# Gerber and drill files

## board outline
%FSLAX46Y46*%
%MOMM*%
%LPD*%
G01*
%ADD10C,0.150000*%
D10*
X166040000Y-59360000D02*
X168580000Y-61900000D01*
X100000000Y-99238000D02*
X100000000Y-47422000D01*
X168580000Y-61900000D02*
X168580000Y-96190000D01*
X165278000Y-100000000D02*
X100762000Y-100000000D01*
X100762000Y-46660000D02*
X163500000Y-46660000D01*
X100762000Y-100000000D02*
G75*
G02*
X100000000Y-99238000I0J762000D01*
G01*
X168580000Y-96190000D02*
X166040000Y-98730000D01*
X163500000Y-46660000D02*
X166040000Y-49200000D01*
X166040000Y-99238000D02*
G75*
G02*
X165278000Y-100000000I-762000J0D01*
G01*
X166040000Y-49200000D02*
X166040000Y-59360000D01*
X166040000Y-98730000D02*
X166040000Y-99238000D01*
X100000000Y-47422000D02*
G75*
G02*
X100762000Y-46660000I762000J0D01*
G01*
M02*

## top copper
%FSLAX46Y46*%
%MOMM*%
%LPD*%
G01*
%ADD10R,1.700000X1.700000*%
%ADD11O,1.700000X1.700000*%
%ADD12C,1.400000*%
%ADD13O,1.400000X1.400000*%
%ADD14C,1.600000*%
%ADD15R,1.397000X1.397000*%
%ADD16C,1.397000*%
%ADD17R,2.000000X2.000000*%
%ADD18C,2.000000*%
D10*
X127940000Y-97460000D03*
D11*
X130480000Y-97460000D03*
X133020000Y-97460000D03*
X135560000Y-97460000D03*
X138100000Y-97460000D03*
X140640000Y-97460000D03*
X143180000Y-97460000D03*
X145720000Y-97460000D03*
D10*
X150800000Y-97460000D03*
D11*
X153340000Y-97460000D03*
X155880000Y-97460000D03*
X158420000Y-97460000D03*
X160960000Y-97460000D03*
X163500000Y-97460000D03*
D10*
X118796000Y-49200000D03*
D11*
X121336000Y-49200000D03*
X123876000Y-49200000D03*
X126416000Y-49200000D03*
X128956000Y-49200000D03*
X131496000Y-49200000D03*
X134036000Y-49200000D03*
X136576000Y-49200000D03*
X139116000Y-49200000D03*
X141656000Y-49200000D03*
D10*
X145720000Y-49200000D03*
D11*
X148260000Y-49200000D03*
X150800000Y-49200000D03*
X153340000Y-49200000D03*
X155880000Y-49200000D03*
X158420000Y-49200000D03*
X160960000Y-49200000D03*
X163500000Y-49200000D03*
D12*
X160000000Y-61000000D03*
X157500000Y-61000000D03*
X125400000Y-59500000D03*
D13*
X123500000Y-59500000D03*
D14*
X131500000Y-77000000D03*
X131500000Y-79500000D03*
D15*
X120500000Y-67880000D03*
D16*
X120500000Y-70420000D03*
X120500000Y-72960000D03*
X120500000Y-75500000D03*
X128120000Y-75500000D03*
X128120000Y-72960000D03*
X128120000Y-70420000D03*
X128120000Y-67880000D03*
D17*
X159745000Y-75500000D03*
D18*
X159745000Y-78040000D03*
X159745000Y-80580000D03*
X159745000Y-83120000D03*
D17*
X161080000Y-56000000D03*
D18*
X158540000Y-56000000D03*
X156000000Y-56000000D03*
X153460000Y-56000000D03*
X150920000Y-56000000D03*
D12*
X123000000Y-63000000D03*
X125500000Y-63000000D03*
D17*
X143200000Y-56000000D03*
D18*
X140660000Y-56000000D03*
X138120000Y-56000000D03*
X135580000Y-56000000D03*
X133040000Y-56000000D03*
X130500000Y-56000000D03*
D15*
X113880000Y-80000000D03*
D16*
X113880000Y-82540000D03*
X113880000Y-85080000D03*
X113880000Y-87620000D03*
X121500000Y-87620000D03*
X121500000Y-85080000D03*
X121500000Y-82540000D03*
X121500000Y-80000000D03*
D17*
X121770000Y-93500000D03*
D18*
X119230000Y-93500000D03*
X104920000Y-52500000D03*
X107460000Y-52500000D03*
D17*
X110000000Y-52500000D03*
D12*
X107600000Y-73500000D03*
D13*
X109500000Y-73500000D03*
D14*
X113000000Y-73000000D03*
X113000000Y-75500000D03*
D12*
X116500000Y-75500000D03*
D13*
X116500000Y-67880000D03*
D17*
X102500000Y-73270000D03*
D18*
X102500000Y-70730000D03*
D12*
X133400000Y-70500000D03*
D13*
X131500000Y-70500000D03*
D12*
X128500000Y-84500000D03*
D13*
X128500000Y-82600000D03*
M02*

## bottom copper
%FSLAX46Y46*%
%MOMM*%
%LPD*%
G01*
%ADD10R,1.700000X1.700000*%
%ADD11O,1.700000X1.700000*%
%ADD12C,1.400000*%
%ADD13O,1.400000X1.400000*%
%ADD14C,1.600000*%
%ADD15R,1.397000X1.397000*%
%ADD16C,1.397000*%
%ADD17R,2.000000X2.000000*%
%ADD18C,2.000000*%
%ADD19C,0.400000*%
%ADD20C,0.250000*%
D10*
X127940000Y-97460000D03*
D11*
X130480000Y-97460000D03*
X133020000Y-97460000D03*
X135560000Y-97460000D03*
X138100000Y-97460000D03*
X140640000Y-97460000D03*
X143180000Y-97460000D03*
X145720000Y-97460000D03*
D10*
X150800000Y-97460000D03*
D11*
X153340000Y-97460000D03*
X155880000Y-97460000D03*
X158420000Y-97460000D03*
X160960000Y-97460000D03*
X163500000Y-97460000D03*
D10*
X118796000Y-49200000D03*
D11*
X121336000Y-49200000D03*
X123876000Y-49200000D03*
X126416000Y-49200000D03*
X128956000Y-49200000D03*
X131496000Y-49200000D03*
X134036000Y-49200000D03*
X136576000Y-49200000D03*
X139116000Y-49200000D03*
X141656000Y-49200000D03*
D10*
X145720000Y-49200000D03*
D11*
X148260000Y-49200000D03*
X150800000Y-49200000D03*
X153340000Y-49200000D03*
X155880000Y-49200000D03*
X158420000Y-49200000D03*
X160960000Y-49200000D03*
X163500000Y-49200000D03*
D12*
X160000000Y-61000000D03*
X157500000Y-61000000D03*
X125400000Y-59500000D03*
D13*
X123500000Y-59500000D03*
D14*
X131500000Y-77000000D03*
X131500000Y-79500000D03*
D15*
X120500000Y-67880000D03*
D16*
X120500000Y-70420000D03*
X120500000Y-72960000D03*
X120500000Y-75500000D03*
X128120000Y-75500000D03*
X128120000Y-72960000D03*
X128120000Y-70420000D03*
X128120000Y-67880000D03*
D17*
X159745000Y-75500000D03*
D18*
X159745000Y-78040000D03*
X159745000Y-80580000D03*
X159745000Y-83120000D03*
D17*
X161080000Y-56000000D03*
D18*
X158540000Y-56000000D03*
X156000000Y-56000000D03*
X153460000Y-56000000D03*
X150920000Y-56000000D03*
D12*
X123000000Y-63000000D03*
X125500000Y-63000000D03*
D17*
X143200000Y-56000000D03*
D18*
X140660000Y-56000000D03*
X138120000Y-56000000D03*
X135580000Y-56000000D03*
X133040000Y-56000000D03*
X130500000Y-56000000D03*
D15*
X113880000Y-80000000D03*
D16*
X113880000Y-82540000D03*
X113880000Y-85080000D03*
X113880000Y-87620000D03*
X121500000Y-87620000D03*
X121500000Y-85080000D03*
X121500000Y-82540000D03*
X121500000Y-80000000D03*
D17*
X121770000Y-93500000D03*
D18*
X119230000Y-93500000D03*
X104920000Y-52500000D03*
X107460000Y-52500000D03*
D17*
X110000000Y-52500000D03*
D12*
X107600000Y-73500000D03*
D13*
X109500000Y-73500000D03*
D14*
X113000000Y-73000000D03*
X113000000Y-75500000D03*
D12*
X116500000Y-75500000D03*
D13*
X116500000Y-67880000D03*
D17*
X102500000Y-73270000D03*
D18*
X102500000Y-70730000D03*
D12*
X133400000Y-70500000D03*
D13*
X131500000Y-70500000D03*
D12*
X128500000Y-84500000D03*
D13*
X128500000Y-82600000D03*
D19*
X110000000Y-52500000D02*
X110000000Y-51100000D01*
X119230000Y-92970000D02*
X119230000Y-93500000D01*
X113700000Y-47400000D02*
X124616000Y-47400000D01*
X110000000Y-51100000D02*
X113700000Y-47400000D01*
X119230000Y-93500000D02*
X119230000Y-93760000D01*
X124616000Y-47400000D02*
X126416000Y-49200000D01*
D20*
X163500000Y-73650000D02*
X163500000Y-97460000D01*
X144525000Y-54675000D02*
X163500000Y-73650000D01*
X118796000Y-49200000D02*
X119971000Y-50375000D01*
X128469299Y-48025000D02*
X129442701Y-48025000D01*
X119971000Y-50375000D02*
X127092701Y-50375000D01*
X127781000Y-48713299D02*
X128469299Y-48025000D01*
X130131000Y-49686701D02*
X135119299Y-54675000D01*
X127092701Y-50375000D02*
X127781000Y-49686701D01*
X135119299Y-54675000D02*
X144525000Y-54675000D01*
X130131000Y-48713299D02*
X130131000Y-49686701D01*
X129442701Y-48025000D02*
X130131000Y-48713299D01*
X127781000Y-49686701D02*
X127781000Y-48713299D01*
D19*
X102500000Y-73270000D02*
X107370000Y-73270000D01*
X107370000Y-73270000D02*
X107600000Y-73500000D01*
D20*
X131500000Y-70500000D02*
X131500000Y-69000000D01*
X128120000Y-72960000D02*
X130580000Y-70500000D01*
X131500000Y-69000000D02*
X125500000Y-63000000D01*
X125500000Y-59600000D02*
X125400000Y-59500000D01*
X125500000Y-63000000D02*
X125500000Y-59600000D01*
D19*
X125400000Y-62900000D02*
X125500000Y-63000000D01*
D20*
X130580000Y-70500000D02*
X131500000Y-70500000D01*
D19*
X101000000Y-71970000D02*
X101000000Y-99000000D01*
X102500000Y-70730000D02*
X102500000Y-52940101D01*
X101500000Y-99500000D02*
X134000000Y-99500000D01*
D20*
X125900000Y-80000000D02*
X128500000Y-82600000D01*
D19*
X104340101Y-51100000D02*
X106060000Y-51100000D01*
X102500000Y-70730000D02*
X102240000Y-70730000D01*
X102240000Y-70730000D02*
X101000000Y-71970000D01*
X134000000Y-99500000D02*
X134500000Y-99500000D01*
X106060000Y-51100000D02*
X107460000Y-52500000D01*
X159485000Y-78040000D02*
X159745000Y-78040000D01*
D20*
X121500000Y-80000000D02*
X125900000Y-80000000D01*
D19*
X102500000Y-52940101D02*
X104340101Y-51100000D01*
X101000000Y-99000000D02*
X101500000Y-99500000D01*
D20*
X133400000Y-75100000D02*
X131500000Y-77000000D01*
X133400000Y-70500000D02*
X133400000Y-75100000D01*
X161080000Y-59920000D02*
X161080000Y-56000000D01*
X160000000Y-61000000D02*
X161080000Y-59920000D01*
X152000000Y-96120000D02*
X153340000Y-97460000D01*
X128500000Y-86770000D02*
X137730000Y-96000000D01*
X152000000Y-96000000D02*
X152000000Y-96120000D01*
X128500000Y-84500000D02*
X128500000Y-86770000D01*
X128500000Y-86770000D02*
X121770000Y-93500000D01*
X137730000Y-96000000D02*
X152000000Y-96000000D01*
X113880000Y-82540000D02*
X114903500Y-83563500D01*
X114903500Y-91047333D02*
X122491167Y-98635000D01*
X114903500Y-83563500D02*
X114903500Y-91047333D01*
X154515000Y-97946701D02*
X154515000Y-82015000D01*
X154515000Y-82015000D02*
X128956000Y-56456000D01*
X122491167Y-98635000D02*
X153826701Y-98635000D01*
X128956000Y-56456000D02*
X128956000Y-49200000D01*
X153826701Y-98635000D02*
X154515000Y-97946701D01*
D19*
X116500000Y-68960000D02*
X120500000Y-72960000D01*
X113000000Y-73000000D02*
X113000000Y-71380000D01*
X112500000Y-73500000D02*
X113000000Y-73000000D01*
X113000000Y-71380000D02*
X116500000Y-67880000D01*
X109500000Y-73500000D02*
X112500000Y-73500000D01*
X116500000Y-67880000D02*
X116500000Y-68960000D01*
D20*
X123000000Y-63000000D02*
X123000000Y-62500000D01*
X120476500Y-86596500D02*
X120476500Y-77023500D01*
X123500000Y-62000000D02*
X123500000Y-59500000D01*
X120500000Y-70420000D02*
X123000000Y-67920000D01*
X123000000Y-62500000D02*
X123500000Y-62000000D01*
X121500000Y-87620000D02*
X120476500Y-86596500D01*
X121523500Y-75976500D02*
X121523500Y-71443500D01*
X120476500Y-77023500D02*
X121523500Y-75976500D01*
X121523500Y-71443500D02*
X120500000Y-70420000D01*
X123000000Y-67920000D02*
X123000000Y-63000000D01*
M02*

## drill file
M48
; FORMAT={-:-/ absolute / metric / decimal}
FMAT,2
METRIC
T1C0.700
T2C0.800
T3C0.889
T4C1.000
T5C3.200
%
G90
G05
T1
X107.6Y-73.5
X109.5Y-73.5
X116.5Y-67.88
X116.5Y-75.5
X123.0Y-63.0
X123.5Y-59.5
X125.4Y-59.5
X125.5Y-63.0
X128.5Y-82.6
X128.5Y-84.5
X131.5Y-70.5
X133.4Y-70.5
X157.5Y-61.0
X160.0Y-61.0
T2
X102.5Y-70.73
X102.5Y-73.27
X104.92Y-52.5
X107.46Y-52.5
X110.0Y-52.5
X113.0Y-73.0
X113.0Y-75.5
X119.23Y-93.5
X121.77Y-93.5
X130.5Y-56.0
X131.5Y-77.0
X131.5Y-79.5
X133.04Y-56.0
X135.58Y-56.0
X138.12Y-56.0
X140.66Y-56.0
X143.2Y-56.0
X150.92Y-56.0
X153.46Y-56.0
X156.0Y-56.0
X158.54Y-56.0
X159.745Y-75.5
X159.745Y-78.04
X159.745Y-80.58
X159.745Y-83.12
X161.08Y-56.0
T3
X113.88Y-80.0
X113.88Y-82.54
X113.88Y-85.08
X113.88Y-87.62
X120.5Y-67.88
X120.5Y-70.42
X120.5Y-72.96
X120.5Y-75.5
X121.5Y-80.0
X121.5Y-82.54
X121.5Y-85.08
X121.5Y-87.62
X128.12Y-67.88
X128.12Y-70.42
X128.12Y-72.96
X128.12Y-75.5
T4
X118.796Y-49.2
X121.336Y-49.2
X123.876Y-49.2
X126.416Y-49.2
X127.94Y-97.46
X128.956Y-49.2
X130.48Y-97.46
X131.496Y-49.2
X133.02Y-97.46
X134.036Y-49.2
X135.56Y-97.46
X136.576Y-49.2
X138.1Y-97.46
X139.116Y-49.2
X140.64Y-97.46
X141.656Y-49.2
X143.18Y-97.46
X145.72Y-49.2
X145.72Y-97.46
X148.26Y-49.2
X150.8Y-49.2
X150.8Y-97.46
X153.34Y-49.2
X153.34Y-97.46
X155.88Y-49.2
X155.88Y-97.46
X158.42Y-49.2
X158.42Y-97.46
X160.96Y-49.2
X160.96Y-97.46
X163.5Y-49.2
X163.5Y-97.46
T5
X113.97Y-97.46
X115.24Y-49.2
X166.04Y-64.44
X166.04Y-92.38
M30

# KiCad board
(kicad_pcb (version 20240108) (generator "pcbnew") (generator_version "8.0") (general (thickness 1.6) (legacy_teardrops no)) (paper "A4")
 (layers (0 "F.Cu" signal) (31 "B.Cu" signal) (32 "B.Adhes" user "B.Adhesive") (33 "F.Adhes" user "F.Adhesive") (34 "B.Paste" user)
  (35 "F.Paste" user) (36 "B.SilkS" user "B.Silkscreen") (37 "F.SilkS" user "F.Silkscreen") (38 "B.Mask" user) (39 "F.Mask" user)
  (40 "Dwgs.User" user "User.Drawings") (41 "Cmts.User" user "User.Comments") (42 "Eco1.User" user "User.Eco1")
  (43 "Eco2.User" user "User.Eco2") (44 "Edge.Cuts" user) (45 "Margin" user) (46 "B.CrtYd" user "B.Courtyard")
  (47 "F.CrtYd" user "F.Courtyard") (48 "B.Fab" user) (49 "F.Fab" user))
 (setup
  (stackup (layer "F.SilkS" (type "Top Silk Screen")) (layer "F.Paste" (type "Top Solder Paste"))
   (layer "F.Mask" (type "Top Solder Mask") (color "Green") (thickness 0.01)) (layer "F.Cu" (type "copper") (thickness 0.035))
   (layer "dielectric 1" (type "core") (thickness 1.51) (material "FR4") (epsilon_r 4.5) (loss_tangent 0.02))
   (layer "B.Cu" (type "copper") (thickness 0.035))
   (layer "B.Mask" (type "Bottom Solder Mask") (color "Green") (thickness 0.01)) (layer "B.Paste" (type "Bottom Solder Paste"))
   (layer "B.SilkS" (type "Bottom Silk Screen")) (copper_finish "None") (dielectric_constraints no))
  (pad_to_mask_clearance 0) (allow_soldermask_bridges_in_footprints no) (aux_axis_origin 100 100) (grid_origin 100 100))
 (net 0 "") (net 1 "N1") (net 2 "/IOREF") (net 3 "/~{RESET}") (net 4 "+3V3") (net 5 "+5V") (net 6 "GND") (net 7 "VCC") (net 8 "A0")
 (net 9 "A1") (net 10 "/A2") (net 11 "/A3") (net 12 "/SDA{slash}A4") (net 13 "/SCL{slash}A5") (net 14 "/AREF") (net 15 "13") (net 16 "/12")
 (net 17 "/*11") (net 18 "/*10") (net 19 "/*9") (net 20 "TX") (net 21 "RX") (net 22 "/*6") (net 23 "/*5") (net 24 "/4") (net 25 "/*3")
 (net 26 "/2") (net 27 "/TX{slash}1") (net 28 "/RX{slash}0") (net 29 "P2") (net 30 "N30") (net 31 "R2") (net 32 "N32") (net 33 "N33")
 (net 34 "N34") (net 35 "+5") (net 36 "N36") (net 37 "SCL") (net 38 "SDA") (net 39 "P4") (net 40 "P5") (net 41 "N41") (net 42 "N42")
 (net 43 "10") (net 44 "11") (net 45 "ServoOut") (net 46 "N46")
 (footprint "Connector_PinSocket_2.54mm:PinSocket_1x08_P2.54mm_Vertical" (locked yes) (layer "F.Cu") (at 127.94 97.46 90)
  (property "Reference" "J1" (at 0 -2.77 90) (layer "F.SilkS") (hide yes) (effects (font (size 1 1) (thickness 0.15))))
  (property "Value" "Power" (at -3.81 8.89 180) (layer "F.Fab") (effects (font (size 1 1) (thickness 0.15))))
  (pad "1" thru_hole rect (at 0 0 90) (size 1.7 1.7) (drill 1) (layers "*.Cu" "*.Mask") (remove_unused_layers no) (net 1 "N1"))
  (pad "2" thru_hole oval (at 0 2.54 90) (size 1.7 1.7) (drill 1) (layers "*.Cu" "*.Mask") (remove_unused_layers no) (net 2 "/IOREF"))
  (pad "3" thru_hole oval (at 0 5.08 90) (size 1.7 1.7) (drill 1) (layers "*.Cu" "*.Mask") (remove_unused_layers no) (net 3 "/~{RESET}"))
  (pad "4" thru_hole oval (at 0 7.62 90) (size 1.7 1.7) (drill 1) (layers "*.Cu" "*.Mask") (remove_unused_layers no) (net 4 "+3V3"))
  (pad "5" thru_hole oval (at 0 10.16 90) (size 1.7 1.7) (drill 1) (layers "*.Cu" "*.Mask") (remove_unused_layers no) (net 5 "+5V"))
  (pad "6" thru_hole oval (at 0 12.7 90) (size 1.7 1.7) (drill 1) (layers "*.Cu" "*.Mask") (remove_unused_layers no) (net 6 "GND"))
  (pad "7" thru_hole oval (at 0 15.24 90) (size 1.7 1.7) (drill 1) (layers "*.Cu" "*.Mask") (remove_unused_layers no) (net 6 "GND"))
  (pad "8" thru_hole oval (at 0 17.78 90) (size 1.7 1.7) (drill 1) (layers "*.Cu" "*.Mask") (remove_unused_layers no) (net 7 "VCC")))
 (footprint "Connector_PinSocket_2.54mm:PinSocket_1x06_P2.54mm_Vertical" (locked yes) (layer "F.Cu") (at 150.8 97.46 90)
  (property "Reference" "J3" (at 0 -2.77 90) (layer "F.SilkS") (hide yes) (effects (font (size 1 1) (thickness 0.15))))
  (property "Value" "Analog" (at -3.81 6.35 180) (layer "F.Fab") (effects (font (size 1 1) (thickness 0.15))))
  (pad "1" thru_hole rect (at 0 0 90) (size 1.7 1.7) (drill 1) (layers "*.Cu" "*.Mask") (remove_unused_layers no) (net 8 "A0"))
  (pad "2" thru_hole oval (at 0 2.54 90) (size 1.7 1.7) (drill 1) (layers "*.Cu" "*.Mask") (remove_unused_layers no) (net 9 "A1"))
  (pad "3" thru_hole oval (at 0 5.08 90) (size 1.7 1.7) (drill 1) (layers "*.Cu" "*.Mask") (remove_unused_layers no) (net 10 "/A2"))
  (pad "4" thru_hole oval (at 0 7.62 90) (size 1.7 1.7) (drill 1) (layers "*.Cu" "*.Mask") (remove_unused_layers no) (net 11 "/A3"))
  (pad "5" thru_hole oval (at 0 10.16 90) (size 1.7 1.7) (drill 1) (layers "*.Cu" "*.Mask") (remove_unused_layers no)
   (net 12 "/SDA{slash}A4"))
  (pad "6" thru_hole oval (at 0 12.7 90) (size 1.7 1.7) (drill 1) (layers "*.Cu" "*.Mask") (remove_unused_layers no)
   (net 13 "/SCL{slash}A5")))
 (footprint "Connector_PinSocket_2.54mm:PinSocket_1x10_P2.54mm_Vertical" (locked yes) (layer "F.Cu") (at 118.796 49.2 90)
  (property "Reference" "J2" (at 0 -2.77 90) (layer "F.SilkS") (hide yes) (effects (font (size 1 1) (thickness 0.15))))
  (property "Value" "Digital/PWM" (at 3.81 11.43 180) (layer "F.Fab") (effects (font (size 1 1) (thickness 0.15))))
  (pad "1" thru_hole rect (at 0 0 90) (size 1.7 1.7) (drill 1) (layers "*.Cu" "*.Mask") (remove_unused_layers no) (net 13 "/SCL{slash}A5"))
  (pad "2" thru_hole oval (at 0 2.54 90) (size 1.7 1.7) (drill 1) (layers "*.Cu" "*.Mask") (remove_unused_layers no)
   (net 12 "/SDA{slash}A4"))
  (pad "3" thru_hole oval (at 0 5.08 90) (size 1.7 1.7) (drill 1) (layers "*.Cu" "*.Mask") (remove_unused_layers no) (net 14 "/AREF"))
  (pad "4" thru_hole oval (at 0 7.62 90) (size 1.7 1.7) (drill 1) (layers "*.Cu" "*.Mask") (remove_unused_layers no) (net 6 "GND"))
  (pad "5" thru_hole oval (at 0 10.16 90) (size 1.7 1.7) (drill 1) (layers "*.Cu" "*.Mask") (remove_unused_layers no) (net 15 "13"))
  (pad "6" thru_hole oval (at 0 12.7 90) (size 1.7 1.7) (drill 1) (layers "*.Cu" "*.Mask") (remove_unused_layers no) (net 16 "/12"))
  (pad "7" thru_hole oval (at 0 15.24 90) (size 1.7 1.7) (drill 1) (layers "*.Cu" "*.Mask") (remove_unused_layers no) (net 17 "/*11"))
  (pad "8" thru_hole oval (at 0 17.78 90) (size 1.7 1.7) (drill 1) (layers "*.Cu" "*.Mask") (remove_unused_layers no) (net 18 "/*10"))
  (pad "9" thru_hole oval (at 0 20.32 90) (size 1.7 1.7) (drill 1) (layers "*.Cu" "*.Mask") (remove_unused_layers no) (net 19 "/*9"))
  (pad "10" thru_hole oval (at 0 22.86 90) (size 1.7 1.7) (drill 1) (layers "*.Cu" "*.Mask") (remove_unused_layers no) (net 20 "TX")))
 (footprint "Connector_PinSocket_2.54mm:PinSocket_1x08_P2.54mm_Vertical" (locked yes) (layer "F.Cu") (at 145.72 49.2 90)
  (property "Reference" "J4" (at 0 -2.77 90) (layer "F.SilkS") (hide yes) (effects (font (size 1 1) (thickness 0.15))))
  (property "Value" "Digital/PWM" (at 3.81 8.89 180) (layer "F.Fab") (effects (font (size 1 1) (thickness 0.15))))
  (pad "1" thru_hole rect (at 0 0 90) (size 1.7 1.7) (drill 1) (layers "*.Cu" "*.Mask") (remove_unused_layers no) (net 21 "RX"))
  (pad "2" thru_hole oval (at 0 2.54 90) (size 1.7 1.7) (drill 1) (layers "*.Cu" "*.Mask") (remove_unused_layers no) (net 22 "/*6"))
  (pad "3" thru_hole oval (at 0 5.08 90) (size 1.7 1.7) (drill 1) (layers "*.Cu" "*.Mask") (remove_unused_layers no) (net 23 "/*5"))
  (pad "4" thru_hole oval (at 0 7.62 90) (size 1.7 1.7) (drill 1) (layers "*.Cu" "*.Mask") (remove_unused_layers no) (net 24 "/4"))
  (pad "5" thru_hole oval (at 0 10.16 90) (size 1.7 1.7) (drill 1) (layers "*.Cu" "*.Mask") (remove_unused_layers no) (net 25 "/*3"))
  (pad "6" thru_hole oval (at 0 12.7 90) (size 1.7 1.7) (drill 1) (layers "*.Cu" "*.Mask") (remove_unused_layers no) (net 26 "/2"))
  (pad "7" thru_hole oval (at 0 15.24 90) (size 1.7 1.7) (drill 1) (layers "*.Cu" "*.Mask") (remove_unused_layers no) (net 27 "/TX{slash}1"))
  (pad "8" thru_hole oval (at 0 17.78 90) (size 1.7 1.7) (drill 1) (layers "*.Cu" "*.Mask") (remove_unused_layers no) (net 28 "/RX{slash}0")))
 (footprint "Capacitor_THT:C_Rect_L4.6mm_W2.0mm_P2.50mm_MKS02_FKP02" (layer "F.Cu") (at 160 61 180)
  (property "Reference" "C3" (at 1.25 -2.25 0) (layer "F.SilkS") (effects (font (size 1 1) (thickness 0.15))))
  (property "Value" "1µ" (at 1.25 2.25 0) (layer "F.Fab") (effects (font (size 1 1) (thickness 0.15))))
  (pad "1" thru_hole circle (at 0 0 180) (size 1.4 1.4) (drill 0.7) (layers "*.Cu" "*.Mask") (remove_unused_layers no) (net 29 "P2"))
  (pad "2" thru_hole circle (at 2.5 0 180) (size 1.4 1.4) (drill 0.7) (layers "*.Cu" "*.Mask") (remove_unused_layers no) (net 6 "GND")))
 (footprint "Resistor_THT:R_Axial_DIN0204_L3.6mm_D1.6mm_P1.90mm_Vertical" (layer "F.Cu") (at 125.4 59.5 180)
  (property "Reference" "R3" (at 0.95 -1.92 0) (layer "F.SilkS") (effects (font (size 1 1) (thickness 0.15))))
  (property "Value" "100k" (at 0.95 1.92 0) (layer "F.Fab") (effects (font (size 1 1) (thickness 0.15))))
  (pad "1" thru_hole circle (at 0 0 180) (size 1.4 1.4) (drill 0.7) (layers "*.Cu" "*.Mask") (remove_unused_layers no) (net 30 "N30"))
  (pad "2" thru_hole oval (at 1.9 0 180) (size 1.4 1.4) (drill 0.7) (layers "*.Cu" "*.Mask") (remove_unused_layers no) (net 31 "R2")))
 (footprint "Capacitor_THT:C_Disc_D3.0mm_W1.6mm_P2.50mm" (layer "F.Cu") (at 131.5 77 -90)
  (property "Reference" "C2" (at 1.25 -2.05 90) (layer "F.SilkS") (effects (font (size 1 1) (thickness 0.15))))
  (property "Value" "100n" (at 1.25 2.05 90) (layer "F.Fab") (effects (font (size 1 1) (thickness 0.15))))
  (pad "1" thru_hole circle (at 0 0 270) (size 1.6 1.6) (drill 0.8) (layers "*.Cu" "*.Mask") (remove_unused_layers no) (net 8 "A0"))
  (pad "2" thru_hole circle (at 2.5 0 270) (size 1.6 1.6) (drill 0.8) (layers "*.Cu" "*.Mask") (remove_unused_layers no) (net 6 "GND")))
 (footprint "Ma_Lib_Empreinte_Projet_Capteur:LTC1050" (layer "F.Cu") (at 128.12 75.5)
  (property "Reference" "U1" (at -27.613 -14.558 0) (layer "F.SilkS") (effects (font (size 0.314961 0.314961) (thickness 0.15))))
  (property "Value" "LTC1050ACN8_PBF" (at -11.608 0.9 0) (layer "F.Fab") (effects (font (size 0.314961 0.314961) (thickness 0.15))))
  (pad "1" thru_hole rect (at -7.62 -7.62) (size 1.397 1.397) (drill 0.889) (layers "*.Cu" "*.Mask") (remove_unused_layers no)
   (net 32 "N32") (solder_mask_margin 0.102))
  (pad "2" thru_hole circle (at -7.62 -5.08) (size 1.397 1.397) (drill 0.889) (layers "*.Cu" "*.Mask") (remove_unused_layers no)
   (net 31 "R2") (solder_mask_margin 0.102))
  (pad "3" thru_hole circle (at -7.62 -2.54) (size 1.397 1.397) (drill 0.889) (layers "*.Cu" "*.Mask") (remove_unused_layers no)
   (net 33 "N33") (solder_mask_margin 0.102))
  (pad "4" thru_hole circle (at -7.62 0) (size 1.397 1.397) (drill 0.889) (layers "*.Cu" "*.Mask") (remove_unused_layers no) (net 6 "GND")
   (solder_mask_margin 0.102))
  (pad "5" thru_hole circle (at 0 0) (size 1.397 1.397) (drill 0.889) (layers "*.Cu" "*.Mask") (remove_unused_layers no) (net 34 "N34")
   (solder_mask_margin 0.102))
  (pad "6" thru_hole circle (at 0 -2.54) (size 1.397 1.397) (drill 0.889) (layers "*.Cu" "*.Mask") (remove_unused_layers no) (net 30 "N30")
   (solder_mask_margin 0.102))
  (pad "7" thru_hole circle (at 0 -5.08) (size 1.397 1.397) (drill 0.889) (layers "*.Cu" "*.Mask") (remove_unused_layers no) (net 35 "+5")
   (solder_mask_margin 0.102))
  (pad "8" thru_hole circle (at 0 -7.62) (size 1.397 1.397) (drill 0.889) (layers "*.Cu" "*.Mask") (remove_unused_layers no) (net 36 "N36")
   (solder_mask_margin 0.102)))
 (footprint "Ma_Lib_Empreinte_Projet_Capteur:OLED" (layer "F.Cu") (at 159.745 79.31 -90)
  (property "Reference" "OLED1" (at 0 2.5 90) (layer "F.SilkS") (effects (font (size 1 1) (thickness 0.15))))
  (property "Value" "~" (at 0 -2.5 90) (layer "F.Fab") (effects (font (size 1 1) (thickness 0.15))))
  (pad "1" thru_hole rect (at -3.81 0 270) (size 2 2) (drill 0.8) (layers "*.Cu" "*.Mask") (remove_unused_layers no) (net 6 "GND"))
  (pad "2" thru_hole circle (at -1.27 0 270) (size 2 2) (drill 0.8) (layers "*.Cu" "*.Mask") (remove_unused_layers no) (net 35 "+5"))
  (pad "3" thru_hole circle (at 1.27 0 270) (size 2 2) (drill 0.8) (layers "*.Cu" "*.Mask") (remove_unused_layers no) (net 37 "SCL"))
  (pad "4" thru_hole circle (at 3.81 0 270) (size 2 2) (drill 0.8) (layers "*.Cu" "*.Mask") (remove_unused_layers no) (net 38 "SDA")))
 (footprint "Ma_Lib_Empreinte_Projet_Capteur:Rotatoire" (layer "F.Cu") (at 156 56 180)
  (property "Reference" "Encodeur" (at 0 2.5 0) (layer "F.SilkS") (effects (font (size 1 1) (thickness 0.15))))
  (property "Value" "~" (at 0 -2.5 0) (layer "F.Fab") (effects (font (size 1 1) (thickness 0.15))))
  (pad "1" thru_hole rect (at -5.08 0 180) (size 2 2) (drill 0.8) (layers "*.Cu" "*.Mask") (remove_unused_layers no) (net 29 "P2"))
  (pad "2" thru_hole circle (at -2.54 0 180) (size 2 2) (drill 0.8) (layers "*.Cu" "*.Mask") (remove_unused_layers no) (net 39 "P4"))
  (pad "3" thru_hole circle (at 0 0 180) (size 2 2) (drill 0.8) (layers "*.Cu" "*.Mask") (remove_unused_layers no) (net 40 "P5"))
  (pad "4" thru_hole circle (at 2.54 0 180) (size 2 2) (drill 0.8) (layers "*.Cu" "*.Mask") (remove_unused_layers no) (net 35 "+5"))
  (pad "5" thru_hole circle (at 5.08 0 180) (size 2 2) (drill 0.8) (layers "*.Cu" "*.Mask") (remove_unused_layers no) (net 6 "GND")))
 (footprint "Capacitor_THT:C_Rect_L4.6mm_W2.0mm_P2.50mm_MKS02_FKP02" (layer "F.Cu") (at 123 63)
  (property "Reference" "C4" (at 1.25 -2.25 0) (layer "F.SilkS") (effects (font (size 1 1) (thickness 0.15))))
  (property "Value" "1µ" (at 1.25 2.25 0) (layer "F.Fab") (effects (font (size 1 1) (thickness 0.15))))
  (pad "1" thru_hole circle (at 0 0) (size 1.4 1.4) (drill 0.7) (layers "*.Cu" "*.Mask") (remove_unused_layers no) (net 31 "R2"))
  (pad "2" thru_hole circle (at 2.5 0) (size 1.4 1.4) (drill 0.7) (layers "*.Cu" "*.Mask") (remove_unused_layers no) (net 30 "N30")))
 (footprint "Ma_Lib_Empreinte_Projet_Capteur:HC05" (layer "F.Cu") (at 136.85 56 180)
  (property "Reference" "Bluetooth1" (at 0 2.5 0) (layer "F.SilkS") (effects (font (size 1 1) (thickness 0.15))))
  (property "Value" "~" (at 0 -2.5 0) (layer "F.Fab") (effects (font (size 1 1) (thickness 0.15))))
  (pad "1" thru_hole rect (at -6.35 0 180) (size 2 2) (drill 0.8) (layers "*.Cu" "*.Mask") (remove_unused_layers no) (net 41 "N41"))
  (pad "2" thru_hole circle (at -3.81 0 180) (size 2 2) (drill 0.8) (layers "*.Cu" "*.Mask") (remove_unused_layers no) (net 21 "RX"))
  (pad "3" thru_hole circle (at -1.27 0 180) (size 2 2) (drill 0.8) (layers "*.Cu" "*.Mask") (remove_unused_layers no) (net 20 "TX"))
  (pad "4" thru_hole circle (at 1.27 0 180) (size 2 2) (drill 0.8) (layers "*.Cu" "*.Mask") (remove_unused_layers no) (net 6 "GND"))
  (pad "5" thru_hole circle (at 3.81 0 180) (size 2 2) (drill 0.8) (layers "*.Cu" "*.Mask") (remove_unused_layers no) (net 7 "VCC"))
  (pad "6" thru_hole circle (at 6.35 0 180) (size 2 2) (drill 0.8) (layers "*.Cu" "*.Mask") (remove_unused_layers no) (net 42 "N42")))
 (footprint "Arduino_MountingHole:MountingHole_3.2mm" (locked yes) (layer "F.Cu") (at 115.24 49.2)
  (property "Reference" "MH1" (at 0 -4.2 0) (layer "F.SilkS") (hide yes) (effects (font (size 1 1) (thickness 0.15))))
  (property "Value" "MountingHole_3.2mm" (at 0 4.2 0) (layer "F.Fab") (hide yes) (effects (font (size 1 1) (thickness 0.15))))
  (pad "" np_thru_hole circle (at 0 0) (size 3.2 3.2) (drill 3.2) (layers "*.Cu" "*.Mask")))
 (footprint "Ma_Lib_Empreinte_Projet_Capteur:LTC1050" (layer "F.Cu") (at 121.5 87.62)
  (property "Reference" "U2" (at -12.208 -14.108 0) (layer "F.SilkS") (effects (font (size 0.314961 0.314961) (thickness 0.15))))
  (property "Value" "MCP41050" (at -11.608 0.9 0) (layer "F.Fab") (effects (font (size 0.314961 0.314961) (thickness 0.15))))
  (pad "1" thru_hole rect (at -7.62 -7.62) (size 1.397 1.397) (drill 0.889) (layers "*.Cu" "*.Mask") (remove_unused_layers no) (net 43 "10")
   (solder_mask_margin 0.102))
  (pad "2" thru_hole circle (at -7.62 -5.08) (size 1.397 1.397) (drill 0.889) (layers "*.Cu" "*.Mask") (remove_unused_layers no)
   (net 15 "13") (solder_mask_margin 0.102))
  (pad "3" thru_hole circle (at -7.62 -2.54) (size 1.397 1.397) (drill 0.889) (layers "*.Cu" "*.Mask") (remove_unused_layers no)
   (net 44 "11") (solder_mask_margin 0.102))
  (pad "4" thru_hole circle (at -7.62 0) (size 1.397 1.397) (drill 0.889) (layers "*.Cu" "*.Mask") (remove_unused_layers no) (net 6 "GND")
   (solder_mask_margin 0.102))
  (pad "5" thru_hole circle (at 0 0) (size 1.397 1.397) (drill 0.889) (layers "*.Cu" "*.Mask") (remove_unused_layers no) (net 31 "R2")
   (solder_mask_margin 0.102))
  (pad "6" thru_hole circle (at 0 -2.54) (size 1.397 1.397) (drill 0.889) (layers "*.Cu" "*.Mask") (remove_unused_layers no) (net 6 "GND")
   (solder_mask_margin 0.102))
  (pad "7" thru_hole circle (at 0 -5.08) (size 1.397 1.397) (drill 0.889) (layers "*.Cu" "*.Mask") (remove_unused_layers no) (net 6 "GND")
   (solder_mask_margin 0.102))
  (pad "8" thru_hole circle (at 0 -7.62) (size 1.397 1.397) (drill 0.889) (layers "*.Cu" "*.Mask") (remove_unused_layers no) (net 35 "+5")
   (solder_mask_margin 0.102)))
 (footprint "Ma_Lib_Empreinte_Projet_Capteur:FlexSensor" (layer "F.Cu") (at 120.5 93.5 180)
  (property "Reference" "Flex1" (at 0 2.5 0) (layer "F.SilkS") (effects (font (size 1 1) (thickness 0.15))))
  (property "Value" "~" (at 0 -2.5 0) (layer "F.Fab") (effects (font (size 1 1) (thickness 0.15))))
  (pad "1" thru_hole rect (at -1.27 0 180) (size 2 2) (drill 0.8) (layers "*.Cu" "*.Mask") (remove_unused_layers no) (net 9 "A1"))
  (pad "2" thru_hole circle (at 1.27 0 180) (size 2 2) (drill 0.8) (layers "*.Cu" "*.Mask") (remove_unused_layers no) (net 6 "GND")))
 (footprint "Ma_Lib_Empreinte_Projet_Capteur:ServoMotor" (layer "F.Cu") (at 107.46 52.5)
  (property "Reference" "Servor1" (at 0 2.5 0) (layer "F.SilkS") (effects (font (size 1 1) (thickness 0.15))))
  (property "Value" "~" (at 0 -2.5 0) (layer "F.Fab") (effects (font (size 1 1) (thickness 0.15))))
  (pad "1" thru_hole circle (at -2.54 0) (size 2 2) (drill 0.8) (layers "*.Cu" "*.Mask") (remove_unused_layers no) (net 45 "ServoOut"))
  (pad "2" thru_hole circle (at 0 0) (size 2 2) (drill 0.8) (layers "*.Cu" "*.Mask") (remove_unused_layers no) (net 35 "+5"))
  (pad "3" thru_hole rect (at 2.54 0) (size 2 2) (drill 0.8) (layers "*.Cu" "*.Mask") (remove_unused_layers no) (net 6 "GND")))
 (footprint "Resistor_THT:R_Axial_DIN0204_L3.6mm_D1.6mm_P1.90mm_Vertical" (layer "F.Cu") (at 107.6 73.5)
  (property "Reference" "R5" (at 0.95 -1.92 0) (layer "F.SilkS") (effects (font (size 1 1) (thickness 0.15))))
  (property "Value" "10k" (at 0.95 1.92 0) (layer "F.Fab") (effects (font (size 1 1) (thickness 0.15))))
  (pad "1" thru_hole circle (at 0 0) (size 1.4 1.4) (drill 0.7) (layers "*.Cu" "*.Mask") (remove_unused_layers no) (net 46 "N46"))
  (pad "2" thru_hole oval (at 1.9 0) (size 1.4 1.4) (drill 0.7) (layers "*.Cu" "*.Mask") (remove_unused_layers no) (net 33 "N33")))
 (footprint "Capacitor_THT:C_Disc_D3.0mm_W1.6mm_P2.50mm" (layer "F.Cu") (at 113 73 -90)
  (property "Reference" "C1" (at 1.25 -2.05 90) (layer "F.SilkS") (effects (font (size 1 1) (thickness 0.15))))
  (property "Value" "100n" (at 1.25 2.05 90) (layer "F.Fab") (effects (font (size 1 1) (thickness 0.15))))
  (pad "1" thru_hole circle (at 0 0 270) (size 1.6 1.6) (drill 0.8) (layers "*.Cu" "*.Mask") (remove_unused_layers no) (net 33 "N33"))
  (pad "2" thru_hole circle (at 2.5 0 270) (size 1.6 1.6) (drill 0.8) (layers "*.Cu" "*.Mask") (remove_unused_layers no) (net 6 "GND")))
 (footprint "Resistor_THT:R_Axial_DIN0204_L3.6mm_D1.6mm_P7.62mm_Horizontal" (layer "F.Cu") (at 116.5 75.5 90)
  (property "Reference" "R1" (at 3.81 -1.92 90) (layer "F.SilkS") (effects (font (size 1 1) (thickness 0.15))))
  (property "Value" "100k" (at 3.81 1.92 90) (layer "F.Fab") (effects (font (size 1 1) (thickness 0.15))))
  (pad "1" thru_hole circle (at 0 0 90) (size 1.4 1.4) (drill 0.7) (layers "*.Cu" "*.Mask") (remove_unused_layers no) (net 6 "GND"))
  (pad "2" thru_hole oval (at 7.62 0 90) (size 1.4 1.4) (drill 0.7) (layers "*.Cu" "*.Mask") (remove_unused_layers no) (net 33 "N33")))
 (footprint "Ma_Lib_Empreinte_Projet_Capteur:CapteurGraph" (layer "F.Cu") (at 102.5 72 90)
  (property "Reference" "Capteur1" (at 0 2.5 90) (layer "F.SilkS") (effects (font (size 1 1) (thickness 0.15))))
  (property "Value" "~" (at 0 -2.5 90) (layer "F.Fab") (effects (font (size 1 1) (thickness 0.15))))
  (pad "1" thru_hole rect (at -1.27 0 90) (size 2 2) (drill 0.8) (layers "*.Cu" "*.Mask") (remove_unused_layers no) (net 46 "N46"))
  (pad "2" thru_hole circle (at 1.27 0 90) (size 2 2) (drill 0.8) (layers "*.Cu" "*.Mask") (remove_unused_layers no) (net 35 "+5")))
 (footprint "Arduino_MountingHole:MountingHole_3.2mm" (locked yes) (layer "F.Cu") (at 113.97 97.46)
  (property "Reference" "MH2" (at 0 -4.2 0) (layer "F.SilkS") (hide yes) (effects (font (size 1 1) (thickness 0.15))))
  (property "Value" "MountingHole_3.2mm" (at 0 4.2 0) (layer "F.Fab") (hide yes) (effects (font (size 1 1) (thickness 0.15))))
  (pad "" np_thru_hole circle (at 0 0) (size 3.2 3.2) (drill 3.2) (layers "*.Cu" "*.Mask")))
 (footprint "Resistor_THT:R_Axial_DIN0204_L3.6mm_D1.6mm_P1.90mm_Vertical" (layer "F.Cu") (at 133.4 70.5 180)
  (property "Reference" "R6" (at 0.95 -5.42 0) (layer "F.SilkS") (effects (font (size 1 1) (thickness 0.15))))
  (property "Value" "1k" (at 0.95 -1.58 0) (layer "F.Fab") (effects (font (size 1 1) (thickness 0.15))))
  (pad "1" thru_hole circle (at 0 0 180) (size 1.4 1.4) (drill 0.7) (layers "*.Cu" "*.Mask") (remove_unused_layers no) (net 8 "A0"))
  (pad "2" thru_hole oval (at 1.9 0 180) (size 1.4 1.4) (drill 0.7) (layers "*.Cu" "*.Mask") (remove_unused_layers no) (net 30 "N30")))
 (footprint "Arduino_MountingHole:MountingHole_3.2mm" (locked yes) (layer "F.Cu") (at 166.04 64.44)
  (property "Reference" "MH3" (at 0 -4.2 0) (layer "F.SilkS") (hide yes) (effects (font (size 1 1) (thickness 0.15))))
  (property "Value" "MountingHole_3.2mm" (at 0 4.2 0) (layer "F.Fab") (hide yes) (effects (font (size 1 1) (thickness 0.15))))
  (pad "" np_thru_hole circle (at 0 0) (size 3.2 3.2) (drill 3.2) (layers "*.Cu" "*.Mask")))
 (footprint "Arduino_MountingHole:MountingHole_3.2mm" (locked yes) (layer "F.Cu") (at 166.04 92.38)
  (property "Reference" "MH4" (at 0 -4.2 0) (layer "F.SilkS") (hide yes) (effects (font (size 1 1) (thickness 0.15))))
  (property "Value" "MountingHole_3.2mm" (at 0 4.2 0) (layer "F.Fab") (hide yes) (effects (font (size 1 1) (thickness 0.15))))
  (pad "" np_thru_hole circle (at 0 0) (size 3.2 3.2) (drill 3.2) (layers "*.Cu" "*.Mask")))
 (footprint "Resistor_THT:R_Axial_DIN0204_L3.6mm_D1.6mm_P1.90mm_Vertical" (layer "F.Cu") (at 128.5 84.5 90)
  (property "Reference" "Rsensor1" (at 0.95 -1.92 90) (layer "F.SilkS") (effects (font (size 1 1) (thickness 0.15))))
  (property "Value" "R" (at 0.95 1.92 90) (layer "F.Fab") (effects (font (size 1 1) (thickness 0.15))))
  (pad "1" thru_hole circle (at 0 0 90) (size 1.4 1.4) (drill 0.7) (layers "*.Cu" "*.Mask") (remove_unused_layers no) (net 9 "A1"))
  (pad "2" thru_hole oval (at 1.9 0 90) (size 1.4 1.4) (drill 0.7) (layers "*.Cu" "*.Mask") (remove_unused_layers no) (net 35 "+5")))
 (gr_line (start 166.04 59.36) (end 168.58 61.9) (stroke (width 0.15) (type solid)) (layer "Edge.Cuts"))
 (gr_line (start 100 99.238) (end 100 47.422) (stroke (width 0.15) (type solid)) (layer "Edge.Cuts"))
 (gr_line (start 168.58 61.9) (end 168.58 96.19) (stroke (width 0.15) (type solid)) (layer "Edge.Cuts"))
 (gr_line (start 165.278 100) (end 100.762 100) (stroke (width 0.15) (type solid)) (layer "Edge.Cuts"))
 (gr_line (start 100.762 46.66) (end 163.5 46.66) (stroke (width 0.15) (type solid)) (layer "Edge.Cuts"))
 (gr_arc (start 100.762 100) (mid 100.223185 99.776815) (end 100 99.238) (stroke (width 0.15) (type solid)) (layer "Edge.Cuts"))
 (gr_line (start 168.58 96.19) (end 166.04 98.73) (stroke (width 0.15) (type solid)) (layer "Edge.Cuts"))
 (gr_line (start 163.5 46.66) (end 166.04 49.2) (stroke (width 0.15) (type solid)) (layer "Edge.Cuts"))
 (gr_arc (start 166.04 99.238) (mid 165.816815 99.776815) (end 165.278 100) (stroke (width 0.15) (type solid)) (layer "Edge.Cuts"))
 (gr_line (start 166.04 49.2) (end 166.04 59.36) (stroke (width 0.15) (type solid)) (layer "Edge.Cuts"))
 (gr_line (start 166.04 98.73) (end 166.04 99.238) (stroke (width 0.15) (type solid)) (layer "Edge.Cuts"))
 (gr_arc (start 100 47.422) (mid 100.223185 46.883185) (end 100.762 46.66) (stroke (width 0.15) (type solid)) (layer "Edge.Cuts"))
 (segment (start 110 52.5) (end 110 51.1) (width 0.4) (layer "B.Cu") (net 6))
 (segment (start 119.23 92.97) (end 119.23 93.5) (width 0.4) (layer "B.Cu") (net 6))
 (segment (start 113.7 47.4) (end 124.616 47.4) (width 0.4) (layer "B.Cu") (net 6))
 (segment (start 110 51.1) (end 113.7 47.4) (width 0.4) (layer "B.Cu") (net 6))
 (segment (start 119.23 93.5) (end 119.23 93.76) (width 0.4) (layer "B.Cu") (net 6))
 (segment (start 124.616 47.4) (end 126.416 49.2) (width 0.4) (layer "B.Cu") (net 6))
 (segment (start 163.5 73.65) (end 163.5 97.46) (width 0.25) (layer "B.Cu") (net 13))
 (segment (start 144.525 54.675) (end 163.5 73.65) (width 0.25) (layer "B.Cu") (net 13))
 (segment (start 118.796 49.2) (end 119.971 50.375) (width 0.25) (layer "B.Cu") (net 13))
 (segment (start 128.469299 48.025) (end 129.442701 48.025) (width 0.25) (layer "B.Cu") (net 13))
 (segment (start 119.971 50.375) (end 127.092701 50.375) (width 0.25) (layer "B.Cu") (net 13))
 (segment (start 127.781 48.713299) (end 128.469299 48.025) (width 0.25) (layer "B.Cu") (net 13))
 (segment (start 130.131 49.686701) (end 135.119299 54.675) (width 0.25) (layer "B.Cu") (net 13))
 (segment (start 127.092701 50.375) (end 127.781 49.686701) (width 0.25) (layer "B.Cu") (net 13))
 (segment (start 135.119299 54.675) (end 144.525 54.675) (width 0.25) (layer "B.Cu") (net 13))
 (segment (start 130.131 48.713299) (end 130.131 49.686701) (width 0.25) (layer "B.Cu") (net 13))
 (segment (start 129.442701 48.025) (end 130.131 48.713299) (width 0.25) (layer "B.Cu") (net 13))
 (segment (start 127.781 49.686701) (end 127.781 48.713299) (width 0.25) (layer "B.Cu") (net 13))
 (segment (start 102.5 73.27) (end 107.37 73.27) (width 0.4) (layer "B.Cu") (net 46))
 (segment (start 107.37 73.27) (end 107.6 73.5) (width 0.4) (layer "B.Cu") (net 46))
 (segment (start 131.5 70.5) (end 131.5 69) (width 0.25) (layer "B.Cu") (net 30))
 (segment (start 128.12 72.96) (end 130.58 70.5) (width 0.25) (layer "B.Cu") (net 30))
 (segment (start 131.5 69) (end 125.5 63) (width 0.25) (layer "B.Cu") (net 30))
 (segment (start 125.5 59.6) (end 125.4 59.5) (width 0.25) (layer "B.Cu") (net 30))
 (segment (start 125.5 63) (end 125.5 59.6) (width 0.25) (layer "B.Cu") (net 30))
 (segment (start 125.4 62.9) (end 125.5 63) (width 0.4) (layer "B.Cu") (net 30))
 (segment (start 130.58 70.5) (end 131.5 70.5) (width 0.25) (layer "B.Cu") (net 30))
 (segment (start 101 71.97) (end 101 99) (width 0.4) (layer "B.Cu") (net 35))
 (segment (start 102.5 70.73) (end 102.5 52.940101) (width 0.4) (layer "B.Cu") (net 35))
 (segment (start 101.5 99.5) (end 134 99.5) (width 0.4) (layer "B.Cu") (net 35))
 (segment (start 125.9 80) (end 128.5 82.6) (width 0.25) (layer "B.Cu") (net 35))
 (segment (start 104.340101 51.1) (end 106.06 51.1) (width 0.4) (layer "B.Cu") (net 35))
 (segment (start 102.5 70.73) (end 102.24 70.73) (width 0.4) (layer "B.Cu") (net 35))
 (segment (start 102.24 70.73) (end 101 71.97) (width 0.4) (layer "B.Cu") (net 35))
 (segment (start 134 99.5) (end 134.5 99.5) (width 0.4) (layer "B.Cu") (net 35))
 (segment (start 106.06 51.1) (end 107.46 52.5) (width 0.4) (layer "B.Cu") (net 35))
 (segment (start 159.485 78.04) (end 159.745 78.04) (width 0.4) (layer "B.Cu") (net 35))
 (segment (start 121.5 80) (end 125.9 80) (width 0.25) (layer "B.Cu") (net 35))
 (segment (start 102.5 52.940101) (end 104.340101 51.1) (width 0.4) (layer "B.Cu") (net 35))
 (segment (start 101 99) (end 101.5 99.5) (width 0.4) (layer "B.Cu") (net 35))
 (segment (start 133.4 75.1) (end 131.5 77) (width 0.25) (layer "B.Cu") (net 8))
 (segment (start 133.4 70.5) (end 133.4 75.1) (width 0.25) (layer "B.Cu") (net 8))
 (segment (start 161.08 59.92) (end 161.08 56) (width 0.25) (layer "B.Cu") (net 29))
 (segment (start 160 61) (end 161.08 59.92) (width 0.25) (layer "B.Cu") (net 29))
 (segment (start 152 96.12) (end 153.34 97.46) (width 0.25) (layer "B.Cu") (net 9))
 (segment (start 128.5 86.77) (end 137.73 96) (width 0.25) (layer "B.Cu") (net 9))
 (segment (start 152 96) (end 152 96.12) (width 0.25) (layer "B.Cu") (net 9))
 (segment (start 128.5 84.5) (end 128.5 86.77) (width 0.25) (layer "B.Cu") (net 9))
 (segment (start 128.5 86.77) (end 121.77 93.5) (width 0.25) (layer "B.Cu") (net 9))
 (segment (start 137.73 96) (end 152 96) (width 0.25) (layer "B.Cu") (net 9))
 (segment (start 113.88 82.54) (end 114.9035 83.5635) (width 0.25) (layer "B.Cu") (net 15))
 (segment (start 114.9035 91.047333) (end 122.491167 98.635) (width 0.25) (layer "B.Cu") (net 15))
 (segment (start 114.9035 83.5635) (end 114.9035 91.047333) (width 0.25) (layer "B.Cu") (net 15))
 (segment (start 154.515 97.946701) (end 154.515 82.015) (width 0.25) (layer "B.Cu") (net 15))
 (segment (start 154.515 82.015) (end 128.956 56.456) (width 0.25) (layer "B.Cu") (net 15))
 (segment (start 122.491167 98.635) (end 153.826701 98.635) (width 0.25) (layer "B.Cu") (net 15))
 (segment (start 128.956 56.456) (end 128.956 49.2) (width 0.25) (layer "B.Cu") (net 15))
 (segment (start 153.826701 98.635) (end 154.515 97.946701) (width 0.25) (layer "B.Cu") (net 15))
 (segment (start 116.5 68.96) (end 120.5 72.96) (width 0.4) (layer "B.Cu") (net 33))
 (segment (start 113 73) (end 113 71.38) (width 0.4) (layer "B.Cu") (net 33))
 (segment (start 112.5 73.5) (end 113 73) (width 0.4) (layer "B.Cu") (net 33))
 (segment (start 113 71.38) (end 116.5 67.88) (width 0.4) (layer "B.Cu") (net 33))
 (segment (start 109.5 73.5) (end 112.5 73.5) (width 0.4) (layer "B.Cu") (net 33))
 (segment (start 116.5 67.88) (end 116.5 68.96) (width 0.4) (layer "B.Cu") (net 33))
 (segment (start 123 63) (end 123 62.5) (width 0.25) (layer "B.Cu") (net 31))
 (segment (start 120.4765 86.5965) (end 120.4765 77.0235) (width 0.25) (layer "B.Cu") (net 31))
 (segment (start 123.5 62) (end 123.5 59.5) (width 0.25) (layer "B.Cu") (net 31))
 (segment (start 120.5 70.42) (end 123 67.92) (width 0.25) (layer "B.Cu") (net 31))
 (segment (start 123 62.5) (end 123.5 62) (width 0.25) (layer "B.Cu") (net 31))
 (segment (start 121.5 87.62) (end 120.4765 86.5965) (width 0.25) (layer "B.Cu") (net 31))
 (segment (start 121.5235 75.9765) (end 121.5235 71.4435) (width 0.25) (layer "B.Cu") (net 31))
 (segment (start 120.4765 77.0235) (end 121.5235 75.9765) (width 0.25) (layer "B.Cu") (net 31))
 (segment (start 121.5235 71.4435) (end 120.5 70.42) (width 0.25) (layer "B.Cu") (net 31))
 (segment (start 123 67.92) (end 123 63) (width 0.25) (layer "B.Cu") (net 31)))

